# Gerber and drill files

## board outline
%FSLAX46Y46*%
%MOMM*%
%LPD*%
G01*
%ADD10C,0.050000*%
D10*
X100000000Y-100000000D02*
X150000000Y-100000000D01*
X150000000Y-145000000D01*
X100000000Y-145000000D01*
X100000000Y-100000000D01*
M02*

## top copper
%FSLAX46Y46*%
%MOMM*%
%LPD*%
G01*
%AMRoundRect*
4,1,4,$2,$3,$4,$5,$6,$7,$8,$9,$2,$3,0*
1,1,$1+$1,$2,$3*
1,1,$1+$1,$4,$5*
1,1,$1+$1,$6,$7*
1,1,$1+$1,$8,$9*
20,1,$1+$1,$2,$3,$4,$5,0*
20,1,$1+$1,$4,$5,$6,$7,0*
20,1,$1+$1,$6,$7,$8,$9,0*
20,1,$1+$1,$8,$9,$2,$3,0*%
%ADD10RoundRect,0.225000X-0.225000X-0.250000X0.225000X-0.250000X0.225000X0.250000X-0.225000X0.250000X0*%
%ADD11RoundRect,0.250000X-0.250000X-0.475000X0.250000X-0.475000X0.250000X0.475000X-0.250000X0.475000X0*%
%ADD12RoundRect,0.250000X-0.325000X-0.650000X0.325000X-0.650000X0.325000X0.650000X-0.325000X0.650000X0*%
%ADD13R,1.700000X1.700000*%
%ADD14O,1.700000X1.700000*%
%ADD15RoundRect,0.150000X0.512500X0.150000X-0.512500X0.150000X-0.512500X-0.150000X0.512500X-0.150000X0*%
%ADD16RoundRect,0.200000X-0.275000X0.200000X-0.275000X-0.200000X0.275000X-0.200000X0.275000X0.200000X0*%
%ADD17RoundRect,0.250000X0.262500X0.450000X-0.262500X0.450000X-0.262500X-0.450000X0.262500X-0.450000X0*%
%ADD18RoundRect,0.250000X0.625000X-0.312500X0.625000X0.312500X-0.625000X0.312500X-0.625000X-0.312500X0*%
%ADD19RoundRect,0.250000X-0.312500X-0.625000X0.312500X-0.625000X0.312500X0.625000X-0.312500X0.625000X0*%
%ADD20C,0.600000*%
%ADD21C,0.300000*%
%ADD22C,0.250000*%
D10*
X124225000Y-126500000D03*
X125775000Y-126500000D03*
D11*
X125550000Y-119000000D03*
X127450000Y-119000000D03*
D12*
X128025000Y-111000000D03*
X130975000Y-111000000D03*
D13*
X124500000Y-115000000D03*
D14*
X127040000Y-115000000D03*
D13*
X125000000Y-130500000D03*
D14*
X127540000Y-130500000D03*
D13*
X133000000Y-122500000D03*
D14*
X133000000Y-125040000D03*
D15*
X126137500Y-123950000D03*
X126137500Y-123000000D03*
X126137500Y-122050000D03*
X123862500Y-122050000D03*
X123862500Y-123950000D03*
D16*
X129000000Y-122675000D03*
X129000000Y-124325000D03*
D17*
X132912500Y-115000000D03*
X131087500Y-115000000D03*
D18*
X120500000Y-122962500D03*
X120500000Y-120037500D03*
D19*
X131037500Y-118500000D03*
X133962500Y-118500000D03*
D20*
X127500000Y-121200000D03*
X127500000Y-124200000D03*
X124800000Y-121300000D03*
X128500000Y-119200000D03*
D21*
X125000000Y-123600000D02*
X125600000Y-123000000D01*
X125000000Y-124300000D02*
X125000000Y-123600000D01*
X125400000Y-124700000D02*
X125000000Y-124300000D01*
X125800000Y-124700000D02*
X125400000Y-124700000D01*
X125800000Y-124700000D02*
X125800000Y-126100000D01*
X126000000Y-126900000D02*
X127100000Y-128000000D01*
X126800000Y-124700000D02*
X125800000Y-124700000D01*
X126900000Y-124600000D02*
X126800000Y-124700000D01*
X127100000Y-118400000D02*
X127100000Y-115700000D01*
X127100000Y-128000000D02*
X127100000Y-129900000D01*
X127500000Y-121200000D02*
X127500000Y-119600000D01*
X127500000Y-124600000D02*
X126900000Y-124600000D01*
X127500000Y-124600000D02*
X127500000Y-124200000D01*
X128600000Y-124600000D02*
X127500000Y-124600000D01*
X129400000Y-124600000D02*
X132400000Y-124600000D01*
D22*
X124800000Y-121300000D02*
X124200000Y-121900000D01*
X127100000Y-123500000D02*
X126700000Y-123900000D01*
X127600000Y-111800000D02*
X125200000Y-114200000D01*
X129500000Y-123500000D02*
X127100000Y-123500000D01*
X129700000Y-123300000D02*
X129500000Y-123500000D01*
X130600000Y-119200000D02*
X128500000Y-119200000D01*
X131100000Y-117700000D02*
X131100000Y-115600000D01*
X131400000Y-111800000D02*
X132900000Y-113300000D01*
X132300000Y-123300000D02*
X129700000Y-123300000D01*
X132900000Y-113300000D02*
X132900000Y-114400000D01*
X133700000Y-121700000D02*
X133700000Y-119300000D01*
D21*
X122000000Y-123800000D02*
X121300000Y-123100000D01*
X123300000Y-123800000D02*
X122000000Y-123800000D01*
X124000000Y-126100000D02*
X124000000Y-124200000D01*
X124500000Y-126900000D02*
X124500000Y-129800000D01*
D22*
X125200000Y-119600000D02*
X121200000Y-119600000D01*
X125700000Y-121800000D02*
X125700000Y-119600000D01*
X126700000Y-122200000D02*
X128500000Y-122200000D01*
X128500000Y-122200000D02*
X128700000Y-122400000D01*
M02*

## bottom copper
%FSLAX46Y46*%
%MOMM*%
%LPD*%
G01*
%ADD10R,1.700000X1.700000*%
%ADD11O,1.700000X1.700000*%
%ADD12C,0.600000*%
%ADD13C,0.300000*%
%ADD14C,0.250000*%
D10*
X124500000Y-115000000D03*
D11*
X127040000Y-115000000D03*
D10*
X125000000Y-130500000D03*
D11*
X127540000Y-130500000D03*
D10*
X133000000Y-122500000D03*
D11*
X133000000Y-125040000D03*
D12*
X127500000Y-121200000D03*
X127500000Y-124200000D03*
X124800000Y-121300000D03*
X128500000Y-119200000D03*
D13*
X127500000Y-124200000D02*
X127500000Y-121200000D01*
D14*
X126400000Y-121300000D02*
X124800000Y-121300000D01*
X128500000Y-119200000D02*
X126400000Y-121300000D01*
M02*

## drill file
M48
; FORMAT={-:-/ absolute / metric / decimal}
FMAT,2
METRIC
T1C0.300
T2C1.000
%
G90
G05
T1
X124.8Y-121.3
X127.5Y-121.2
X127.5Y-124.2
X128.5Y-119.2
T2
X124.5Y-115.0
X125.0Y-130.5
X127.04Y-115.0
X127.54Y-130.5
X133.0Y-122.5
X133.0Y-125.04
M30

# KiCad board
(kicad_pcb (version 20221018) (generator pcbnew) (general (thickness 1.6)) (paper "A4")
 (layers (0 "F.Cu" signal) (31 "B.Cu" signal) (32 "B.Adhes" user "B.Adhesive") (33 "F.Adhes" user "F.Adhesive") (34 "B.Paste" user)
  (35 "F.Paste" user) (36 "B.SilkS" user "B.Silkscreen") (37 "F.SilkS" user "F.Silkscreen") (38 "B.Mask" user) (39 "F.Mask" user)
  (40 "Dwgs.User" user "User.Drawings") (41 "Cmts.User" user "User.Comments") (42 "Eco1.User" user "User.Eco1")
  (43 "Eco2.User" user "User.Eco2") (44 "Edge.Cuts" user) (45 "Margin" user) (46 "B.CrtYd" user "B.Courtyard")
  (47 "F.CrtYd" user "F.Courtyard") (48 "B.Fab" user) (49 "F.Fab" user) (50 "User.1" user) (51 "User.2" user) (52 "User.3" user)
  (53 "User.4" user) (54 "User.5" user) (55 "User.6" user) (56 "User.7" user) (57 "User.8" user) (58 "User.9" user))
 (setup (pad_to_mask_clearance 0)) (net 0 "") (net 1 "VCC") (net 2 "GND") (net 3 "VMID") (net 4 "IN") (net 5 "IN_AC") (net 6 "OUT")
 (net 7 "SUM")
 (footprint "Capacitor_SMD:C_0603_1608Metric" (layer "F.Cu") (at 125 126.5)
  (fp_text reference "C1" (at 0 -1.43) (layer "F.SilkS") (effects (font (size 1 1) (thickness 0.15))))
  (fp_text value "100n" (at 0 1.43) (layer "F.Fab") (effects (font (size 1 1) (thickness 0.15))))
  (pad "1" smd roundrect (at -0.775 0) (size 0.9 0.95) (layers "F.Cu" "F.Paste" "F.Mask") (roundrect_rratio 0.25) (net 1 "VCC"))
  (pad "2" smd roundrect (at 0.775 0) (size 0.9 0.95) (layers "F.Cu" "F.Paste" "F.Mask") (roundrect_rratio 0.25) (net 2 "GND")))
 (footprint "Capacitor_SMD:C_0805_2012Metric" (layer "F.Cu") (at 126.5 119)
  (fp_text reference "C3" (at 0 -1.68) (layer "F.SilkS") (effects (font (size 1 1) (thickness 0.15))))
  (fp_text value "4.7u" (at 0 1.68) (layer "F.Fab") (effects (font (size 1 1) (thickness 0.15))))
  (pad "1" smd roundrect (at -0.95 0) (size 1 1.45) (layers "F.Cu" "F.Paste" "F.Mask") (roundrect_rratio 0.25) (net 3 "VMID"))
  (pad "2" smd roundrect (at 0.95 0) (size 1 1.45) (layers "F.Cu" "F.Paste" "F.Mask") (roundrect_rratio 0.25) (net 2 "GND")))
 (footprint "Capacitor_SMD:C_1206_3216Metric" (layer "F.Cu") (at 129.5 111)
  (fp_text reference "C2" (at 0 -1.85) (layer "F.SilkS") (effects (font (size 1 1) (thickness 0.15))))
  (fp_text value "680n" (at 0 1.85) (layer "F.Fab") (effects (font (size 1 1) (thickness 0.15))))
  (pad "1" smd roundrect (at -1.475 0) (size 1.15 1.8) (layers "F.Cu" "F.Paste" "F.Mask") (roundrect_rratio 0.217391) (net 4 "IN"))
  (pad "2" smd roundrect (at 1.475 0) (size 1.15 1.8) (layers "F.Cu" "F.Paste" "F.Mask") (roundrect_rratio 0.217391) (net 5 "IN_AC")))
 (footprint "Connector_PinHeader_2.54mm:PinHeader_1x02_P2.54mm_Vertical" (layer "F.Cu") (at 124.5 115 90)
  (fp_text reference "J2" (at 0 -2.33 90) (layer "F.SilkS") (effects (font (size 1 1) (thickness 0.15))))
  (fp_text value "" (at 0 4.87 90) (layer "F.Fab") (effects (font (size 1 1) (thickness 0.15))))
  (pad "1" thru_hole rect (at 0 0 90) (size 1.7 1.7) (drill 1) (layers "*.Cu" "*.Mask") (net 4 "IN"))
  (pad "2" thru_hole oval (at 0 2.54 90) (size 1.7 1.7) (drill 1) (layers "*.Cu" "*.Mask") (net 2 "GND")))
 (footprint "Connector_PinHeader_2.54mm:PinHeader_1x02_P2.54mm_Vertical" (layer "F.Cu") (at 125 130.5 90)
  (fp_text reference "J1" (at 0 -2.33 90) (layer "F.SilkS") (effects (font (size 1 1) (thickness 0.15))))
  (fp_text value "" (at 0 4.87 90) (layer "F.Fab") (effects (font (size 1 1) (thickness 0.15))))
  (pad "1" thru_hole rect (at 0 0 90) (size 1.7 1.7) (drill 1) (layers "*.Cu" "*.Mask") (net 1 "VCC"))
  (pad "2" thru_hole oval (at 0 2.54 90) (size 1.7 1.7) (drill 1) (layers "*.Cu" "*.Mask") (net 2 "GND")))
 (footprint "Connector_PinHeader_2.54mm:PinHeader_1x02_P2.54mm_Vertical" (layer "F.Cu") (at 133 122.5)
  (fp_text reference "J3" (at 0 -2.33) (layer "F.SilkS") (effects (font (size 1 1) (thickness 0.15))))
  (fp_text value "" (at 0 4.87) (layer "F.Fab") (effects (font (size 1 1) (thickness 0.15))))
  (pad "1" thru_hole rect (at 0 0) (size 1.7 1.7) (drill 1) (layers "*.Cu" "*.Mask") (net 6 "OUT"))
  (pad "2" thru_hole oval (at 0 2.54) (size 1.7 1.7) (drill 1) (layers "*.Cu" "*.Mask") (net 2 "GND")))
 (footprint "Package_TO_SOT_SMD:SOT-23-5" (layer "F.Cu") (at 125 123 180)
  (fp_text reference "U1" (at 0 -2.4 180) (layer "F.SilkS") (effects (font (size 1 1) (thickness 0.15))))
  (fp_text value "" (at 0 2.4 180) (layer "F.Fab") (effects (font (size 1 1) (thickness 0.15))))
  (pad "1" smd roundrect (at -1.1375 -0.95 180) (size 1.325 0.6) (layers "F.Cu" "F.Paste" "F.Mask") (roundrect_rratio 0.25) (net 6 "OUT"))
  (pad "2" smd roundrect (at -1.1375 0 180) (size 1.325 0.6) (layers "F.Cu" "F.Paste" "F.Mask") (roundrect_rratio 0.25) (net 2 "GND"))
  (pad "3" smd roundrect (at -1.1375 0.95 180) (size 1.325 0.6) (layers "F.Cu" "F.Paste" "F.Mask") (roundrect_rratio 0.25) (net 3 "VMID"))
  (pad "4" smd roundrect (at 1.1375 0.95 180) (size 1.325 0.6) (layers "F.Cu" "F.Paste" "F.Mask") (roundrect_rratio 0.25) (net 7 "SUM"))
  (pad "5" smd roundrect (at 1.1375 -0.95 180) (size 1.325 0.6) (layers "F.Cu" "F.Paste" "F.Mask") (roundrect_rratio 0.25) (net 1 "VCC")))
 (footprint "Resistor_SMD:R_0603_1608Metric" (layer "F.Cu") (at 129 123.5 -90)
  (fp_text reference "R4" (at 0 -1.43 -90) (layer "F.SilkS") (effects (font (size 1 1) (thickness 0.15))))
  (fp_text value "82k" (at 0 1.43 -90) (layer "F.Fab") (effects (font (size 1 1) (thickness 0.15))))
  (pad "1" smd roundrect (at -0.825 0 270) (size 0.8 0.95) (layers "F.Cu" "F.Paste" "F.Mask") (roundrect_rratio 0.25) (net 3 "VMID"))
  (pad "2" smd roundrect (at 0.825 0 270) (size 0.8 0.95) (layers "F.Cu" "F.Paste" "F.Mask") (roundrect_rratio 0.25) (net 2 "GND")))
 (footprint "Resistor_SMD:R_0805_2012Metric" (layer "F.Cu") (at 132 115 180)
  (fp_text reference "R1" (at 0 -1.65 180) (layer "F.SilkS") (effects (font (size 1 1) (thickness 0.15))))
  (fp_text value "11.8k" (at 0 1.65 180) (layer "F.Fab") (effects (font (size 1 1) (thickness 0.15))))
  (pad "1" smd roundrect (at -0.9125 0 180) (size 1.025 1.4) (layers "F.Cu" "F.Paste" "F.Mask") (roundrect_rratio 0.243902) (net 5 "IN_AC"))
  (pad "2" smd roundrect (at 0.9125 0 180) (size 1.025 1.4) (layers "F.Cu" "F.Paste" "F.Mask") (roundrect_rratio 0.243902) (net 7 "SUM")))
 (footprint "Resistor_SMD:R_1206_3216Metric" (layer "F.Cu") (at 120.5 121.5 90)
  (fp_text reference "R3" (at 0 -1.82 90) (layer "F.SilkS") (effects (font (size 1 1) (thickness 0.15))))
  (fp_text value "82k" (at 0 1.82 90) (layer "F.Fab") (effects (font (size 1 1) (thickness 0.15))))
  (pad "1" smd roundrect (at -1.4625 0 90) (size 1.125 1.75) (layers "F.Cu" "F.Paste" "F.Mask") (roundrect_rratio 0.222222) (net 1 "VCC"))
  (pad "2" smd roundrect (at 1.4625 0 90) (size 1.125 1.75) (layers "F.Cu" "F.Paste" "F.Mask") (roundrect_rratio 0.222222) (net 3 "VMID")))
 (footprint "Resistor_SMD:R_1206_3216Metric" (layer "F.Cu") (at 132.5 118.5)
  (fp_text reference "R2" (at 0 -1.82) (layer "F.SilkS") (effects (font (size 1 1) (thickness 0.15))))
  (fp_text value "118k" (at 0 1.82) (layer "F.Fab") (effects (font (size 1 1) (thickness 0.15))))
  (pad "1" smd roundrect (at -1.4625 0) (size 1.125 1.75) (layers "F.Cu" "F.Paste" "F.Mask") (roundrect_rratio 0.222222) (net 7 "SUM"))
  (pad "2" smd roundrect (at 1.4625 0) (size 1.125 1.75) (layers "F.Cu" "F.Paste" "F.Mask") (roundrect_rratio 0.222222) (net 6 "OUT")))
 (gr_rect (start 100 100) (end 150 145) (stroke (width 0.05) (type default)) (fill none) (layer "Edge.Cuts"))
 (segment (start 125 123.6) (end 125.6 123) (width 0.3) (layer "F.Cu") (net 2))
 (segment (start 125 124.3) (end 125 123.6) (width 0.3) (layer "F.Cu") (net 2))
 (segment (start 125.4 124.7) (end 125 124.3) (width 0.3) (layer "F.Cu") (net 2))
 (segment (start 125.8 124.7) (end 125.4 124.7) (width 0.3) (layer "F.Cu") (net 2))
 (segment (start 125.8 124.7) (end 125.8 126.1) (width 0.3) (layer "F.Cu") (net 2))
 (segment (start 126 126.9) (end 127.1 128) (width 0.3) (layer "F.Cu") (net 2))
 (segment (start 126.8 124.7) (end 125.8 124.7) (width 0.3) (layer "F.Cu") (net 2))
 (segment (start 126.9 124.6) (end 126.8 124.7) (width 0.3) (layer "F.Cu") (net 2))
 (segment (start 127.1 118.4) (end 127.1 115.7) (width 0.3) (layer "F.Cu") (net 2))
 (segment (start 127.1 128) (end 127.1 129.9) (width 0.3) (layer "F.Cu") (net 2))
 (segment (start 127.5 121.2) (end 127.5 119.6) (width 0.3) (layer "F.Cu") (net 2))
 (segment (start 127.5 124.6) (end 126.9 124.6) (width 0.3) (layer "F.Cu") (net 2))
 (segment (start 127.5 124.6) (end 127.5 124.2) (width 0.3) (layer "F.Cu") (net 2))
 (segment (start 128.6 124.6) (end 127.5 124.6) (width 0.3) (layer "F.Cu") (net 2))
 (segment (start 129.4 124.6) (end 132.4 124.6) (width 0.3) (layer "F.Cu") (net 2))
 (via (at 127.5 121.2) (size 0.6) (drill 0.3) (layers "F.Cu" "B.Cu") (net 2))
 (via (at 127.5 124.2) (size 0.6) (drill 0.3) (layers "F.Cu" "B.Cu") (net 2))
 (segment (start 124.8 121.3) (end 124.2 121.9) (width 0.25) (layer "F.Cu") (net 7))
 (segment (start 127.1 123.5) (end 126.7 123.9) (width 0.25) (layer "F.Cu") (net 6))
 (segment (start 127.5 124.2) (end 127.5 121.2) (width 0.3) (layer "B.Cu") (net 2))
 (segment (start 127.6 111.8) (end 125.2 114.2) (width 0.25) (layer "F.Cu") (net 4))
 (segment (start 129.5 123.5) (end 127.1 123.5) (width 0.25) (layer "F.Cu") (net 6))
 (segment (start 129.7 123.3) (end 129.5 123.5) (width 0.25) (layer "F.Cu") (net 6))
 (segment (start 130.6 119.2) (end 128.5 119.2) (width 0.25) (layer "F.Cu") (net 7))
 (segment (start 131.1 117.7) (end 131.1 115.6) (width 0.25) (layer "F.Cu") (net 7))
 (segment (start 131.4 111.8) (end 132.9 113.3) (width 0.25) (layer "F.Cu") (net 5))
 (segment (start 132.3 123.3) (end 129.7 123.3) (width 0.25) (layer "F.Cu") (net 6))
 (segment (start 132.9 113.3) (end 132.9 114.4) (width 0.25) (layer "F.Cu") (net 5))
 (segment (start 133.7 121.7) (end 133.7 119.3) (width 0.25) (layer "F.Cu") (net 6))
 (via (at 124.8 121.3) (size 0.6) (drill 0.3) (layers "F.Cu" "B.Cu") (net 7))
 (via (at 128.5 119.2) (size 0.6) (drill 0.3) (layers "F.Cu" "B.Cu") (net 7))
 (segment (start 122 123.8) (end 121.3 123.1) (width 0.3) (layer "F.Cu") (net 1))
 (segment (start 123.3 123.8) (end 122 123.8) (width 0.3) (layer "F.Cu") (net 1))
 (segment (start 124 126.1) (end 124 124.2) (width 0.3) (layer "F.Cu") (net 1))
 (segment (start 124.5 126.9) (end 124.5 129.8) (width 0.3) (layer "F.Cu") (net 1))
 (segment (start 125.2 119.6) (end 121.2 119.6) (width 0.25) (layer "F.Cu") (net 3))
 (segment (start 125.7 121.8) (end 125.7 119.6) (width 0.25) (layer "F.Cu") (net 3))
 (segment (start 126.4 121.3) (end 124.8 121.3) (width 0.25) (layer "B.Cu") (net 7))
 (segment (start 126.7 122.2) (end 128.5 122.2) (width 0.25) (layer "F.Cu") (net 3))
 (segment (start 128.5 119.2) (end 126.4 121.3) (width 0.25) (layer "B.Cu") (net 7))
 (segment (start 128.5 122.2) (end 128.7 122.4) (width 0.25) (layer "F.Cu") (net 3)))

